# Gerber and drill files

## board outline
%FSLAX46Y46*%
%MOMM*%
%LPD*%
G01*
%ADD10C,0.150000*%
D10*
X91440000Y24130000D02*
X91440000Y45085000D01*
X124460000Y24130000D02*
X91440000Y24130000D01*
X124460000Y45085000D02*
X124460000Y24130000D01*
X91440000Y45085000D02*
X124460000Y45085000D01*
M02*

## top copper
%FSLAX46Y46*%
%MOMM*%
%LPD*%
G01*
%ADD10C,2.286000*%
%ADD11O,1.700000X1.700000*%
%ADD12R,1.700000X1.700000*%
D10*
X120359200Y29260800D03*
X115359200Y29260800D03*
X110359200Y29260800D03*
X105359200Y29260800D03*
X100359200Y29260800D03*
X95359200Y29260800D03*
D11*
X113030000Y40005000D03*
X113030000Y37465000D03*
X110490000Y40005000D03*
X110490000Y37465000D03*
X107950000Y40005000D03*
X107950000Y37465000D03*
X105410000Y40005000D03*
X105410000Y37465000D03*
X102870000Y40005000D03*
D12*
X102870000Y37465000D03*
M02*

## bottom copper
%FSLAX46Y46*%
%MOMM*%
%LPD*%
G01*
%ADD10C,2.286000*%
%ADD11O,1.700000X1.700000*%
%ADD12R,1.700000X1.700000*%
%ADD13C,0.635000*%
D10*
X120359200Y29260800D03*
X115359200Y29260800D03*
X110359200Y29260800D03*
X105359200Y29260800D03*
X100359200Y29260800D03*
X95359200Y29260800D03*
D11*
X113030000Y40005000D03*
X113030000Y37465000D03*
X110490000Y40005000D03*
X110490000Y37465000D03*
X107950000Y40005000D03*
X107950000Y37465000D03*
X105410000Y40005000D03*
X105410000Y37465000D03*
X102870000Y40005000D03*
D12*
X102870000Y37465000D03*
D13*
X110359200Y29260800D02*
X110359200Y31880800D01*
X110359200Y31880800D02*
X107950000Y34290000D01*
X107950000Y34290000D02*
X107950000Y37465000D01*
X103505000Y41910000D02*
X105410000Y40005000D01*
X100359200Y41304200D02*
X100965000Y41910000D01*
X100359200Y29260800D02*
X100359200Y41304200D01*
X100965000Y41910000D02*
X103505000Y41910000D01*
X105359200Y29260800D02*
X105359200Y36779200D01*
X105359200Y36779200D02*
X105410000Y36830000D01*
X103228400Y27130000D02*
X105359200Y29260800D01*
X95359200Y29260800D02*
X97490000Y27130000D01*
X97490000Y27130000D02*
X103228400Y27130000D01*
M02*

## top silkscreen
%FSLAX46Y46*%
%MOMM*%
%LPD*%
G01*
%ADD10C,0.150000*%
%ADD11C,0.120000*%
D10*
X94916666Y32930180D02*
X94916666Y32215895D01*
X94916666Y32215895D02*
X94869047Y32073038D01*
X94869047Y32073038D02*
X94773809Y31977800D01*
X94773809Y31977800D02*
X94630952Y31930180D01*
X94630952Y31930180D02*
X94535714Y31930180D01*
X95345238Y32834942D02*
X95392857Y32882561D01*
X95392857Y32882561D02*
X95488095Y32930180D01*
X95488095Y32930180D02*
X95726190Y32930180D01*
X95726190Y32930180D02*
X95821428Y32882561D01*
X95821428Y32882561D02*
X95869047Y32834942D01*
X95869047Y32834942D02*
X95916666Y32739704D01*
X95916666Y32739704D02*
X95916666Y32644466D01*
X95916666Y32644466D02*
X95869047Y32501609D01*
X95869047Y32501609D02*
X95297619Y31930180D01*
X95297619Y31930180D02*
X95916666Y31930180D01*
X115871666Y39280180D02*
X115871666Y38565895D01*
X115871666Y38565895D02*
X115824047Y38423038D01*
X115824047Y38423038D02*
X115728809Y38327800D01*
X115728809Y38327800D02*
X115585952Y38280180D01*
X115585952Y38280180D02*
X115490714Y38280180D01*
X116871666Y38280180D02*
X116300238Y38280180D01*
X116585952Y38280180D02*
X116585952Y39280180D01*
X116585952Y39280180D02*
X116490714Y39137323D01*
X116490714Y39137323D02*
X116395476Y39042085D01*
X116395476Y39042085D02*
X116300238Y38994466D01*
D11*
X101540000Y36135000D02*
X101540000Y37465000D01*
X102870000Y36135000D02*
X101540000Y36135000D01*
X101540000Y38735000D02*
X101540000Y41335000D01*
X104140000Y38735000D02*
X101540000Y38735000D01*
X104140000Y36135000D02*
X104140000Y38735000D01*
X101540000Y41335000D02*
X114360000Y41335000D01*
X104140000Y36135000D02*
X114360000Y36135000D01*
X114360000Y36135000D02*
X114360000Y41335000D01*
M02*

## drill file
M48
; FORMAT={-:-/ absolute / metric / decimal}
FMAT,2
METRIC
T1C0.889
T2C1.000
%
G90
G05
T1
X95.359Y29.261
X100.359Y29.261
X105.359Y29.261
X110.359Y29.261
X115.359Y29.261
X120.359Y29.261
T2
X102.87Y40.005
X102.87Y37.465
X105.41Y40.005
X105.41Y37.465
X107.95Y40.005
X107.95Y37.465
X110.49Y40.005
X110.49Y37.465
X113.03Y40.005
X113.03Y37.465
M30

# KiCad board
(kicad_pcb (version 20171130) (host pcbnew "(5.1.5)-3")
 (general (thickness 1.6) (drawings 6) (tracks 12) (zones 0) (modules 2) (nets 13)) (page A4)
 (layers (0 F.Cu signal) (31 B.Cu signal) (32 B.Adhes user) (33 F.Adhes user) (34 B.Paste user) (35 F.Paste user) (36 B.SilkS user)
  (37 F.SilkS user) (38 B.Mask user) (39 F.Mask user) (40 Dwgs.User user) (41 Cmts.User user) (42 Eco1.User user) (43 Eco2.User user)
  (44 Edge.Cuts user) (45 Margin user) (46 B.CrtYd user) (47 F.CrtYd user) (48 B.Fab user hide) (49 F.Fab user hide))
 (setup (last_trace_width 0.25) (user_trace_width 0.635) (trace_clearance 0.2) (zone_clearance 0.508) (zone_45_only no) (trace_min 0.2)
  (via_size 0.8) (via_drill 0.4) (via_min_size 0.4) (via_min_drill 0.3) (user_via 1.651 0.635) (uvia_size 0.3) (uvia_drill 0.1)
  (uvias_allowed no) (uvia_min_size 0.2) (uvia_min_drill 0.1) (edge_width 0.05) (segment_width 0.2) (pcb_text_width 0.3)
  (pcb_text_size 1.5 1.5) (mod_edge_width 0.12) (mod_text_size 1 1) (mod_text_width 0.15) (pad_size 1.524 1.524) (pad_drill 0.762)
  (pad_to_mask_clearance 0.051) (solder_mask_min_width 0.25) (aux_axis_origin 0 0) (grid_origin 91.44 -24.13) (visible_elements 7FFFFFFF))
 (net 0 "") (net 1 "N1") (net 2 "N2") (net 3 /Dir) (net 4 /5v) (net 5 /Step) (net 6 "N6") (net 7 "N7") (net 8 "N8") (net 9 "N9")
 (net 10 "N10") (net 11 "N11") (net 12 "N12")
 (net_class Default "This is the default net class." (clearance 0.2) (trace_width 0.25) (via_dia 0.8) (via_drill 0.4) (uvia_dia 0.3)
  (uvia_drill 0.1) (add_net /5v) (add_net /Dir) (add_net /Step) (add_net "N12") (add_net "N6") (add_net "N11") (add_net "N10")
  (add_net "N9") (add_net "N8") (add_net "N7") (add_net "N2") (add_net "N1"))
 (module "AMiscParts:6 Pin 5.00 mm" (layer F.Cu) (at 107.8592 -29.2608)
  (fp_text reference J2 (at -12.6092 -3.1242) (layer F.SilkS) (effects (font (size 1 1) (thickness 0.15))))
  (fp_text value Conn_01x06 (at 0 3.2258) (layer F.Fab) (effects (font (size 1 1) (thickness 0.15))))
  (pad 6 thru_hole circle (at 12.5 0) (size 2.286 2.286) (drill 0.889) (layers *.Cu *.Mask) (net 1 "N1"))
  (pad 5 thru_hole circle (at 7.5 0) (size 2.286 2.286) (drill 0.889) (layers *.Cu *.Mask) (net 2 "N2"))
  (pad 4 thru_hole circle (at 2.5 0) (size 2.286 2.286) (drill 0.889) (layers *.Cu *.Mask) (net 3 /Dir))
  (pad 3 thru_hole circle (at -2.5 0) (size 2.286 2.286) (drill 0.889) (layers *.Cu *.Mask) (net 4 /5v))
  (pad 2 thru_hole circle (at -7.5 0) (size 2.286 2.286) (drill 0.889) (layers *.Cu *.Mask) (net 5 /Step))
  (pad 1 thru_hole circle (at -12.5 0) (size 2.286 2.286) (drill 0.889) (layers *.Cu *.Mask) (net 4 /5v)))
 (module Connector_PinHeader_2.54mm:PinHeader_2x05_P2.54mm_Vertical (layer F.Cu) (at 102.87 -37.465 90)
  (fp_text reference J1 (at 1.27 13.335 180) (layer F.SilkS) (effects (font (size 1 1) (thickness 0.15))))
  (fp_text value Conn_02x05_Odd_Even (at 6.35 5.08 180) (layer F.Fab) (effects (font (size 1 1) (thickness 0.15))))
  (fp_line (start -1.33 -1.33) (end 0 -1.33) (layer F.SilkS) (width 0.12))
  (fp_line (start -1.33 0) (end -1.33 -1.33) (layer F.SilkS) (width 0.12))
  (fp_line (start 1.27 -1.33) (end 3.87 -1.33) (layer F.SilkS) (width 0.12))
  (fp_line (start 1.27 1.27) (end 1.27 -1.33) (layer F.SilkS) (width 0.12))
  (fp_line (start -1.33 1.27) (end 1.27 1.27) (layer F.SilkS) (width 0.12))
  (fp_line (start 3.87 -1.33) (end 3.87 11.49) (layer F.SilkS) (width 0.12))
  (fp_line (start -1.33 1.27) (end -1.33 11.49) (layer F.SilkS) (width 0.12))
  (fp_line (start -1.33 11.49) (end 3.87 11.49) (layer F.SilkS) (width 0.12))
  (pad 10 thru_hole oval (at 2.54 10.16 90) (size 1.7 1.7) (drill 1) (layers *.Cu *.Mask) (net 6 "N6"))
  (pad 9 thru_hole oval (at 0 10.16 90) (size 1.7 1.7) (drill 1) (layers *.Cu *.Mask) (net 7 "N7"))
  (pad 8 thru_hole oval (at 2.54 7.62 90) (size 1.7 1.7) (drill 1) (layers *.Cu *.Mask) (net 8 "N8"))
  (pad 7 thru_hole oval (at 0 7.62 90) (size 1.7 1.7) (drill 1) (layers *.Cu *.Mask) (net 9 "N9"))
  (pad 6 thru_hole oval (at 2.54 5.08 90) (size 1.7 1.7) (drill 1) (layers *.Cu *.Mask) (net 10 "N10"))
  (pad 5 thru_hole oval (at 0 5.08 90) (size 1.7 1.7) (drill 1) (layers *.Cu *.Mask) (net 3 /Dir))
  (pad 4 thru_hole oval (at 2.54 2.54 90) (size 1.7 1.7) (drill 1) (layers *.Cu *.Mask) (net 5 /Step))
  (pad 3 thru_hole oval (at 0 2.54 90) (size 1.7 1.7) (drill 1) (layers *.Cu *.Mask) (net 4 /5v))
  (pad 2 thru_hole oval (at 2.54 0 90) (size 1.7 1.7) (drill 1) (layers *.Cu *.Mask) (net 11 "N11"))
  (pad 1 thru_hole rect (at 0 0 90) (size 1.7 1.7) (drill 1) (layers *.Cu *.Mask) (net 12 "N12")))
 (gr_line (start 91.44 -24.13) (end 91.44 -45.085) (layer Edge.Cuts) (width 0.15))
 (gr_line (start 124.46 -24.13) (end 91.44 -24.13) (layer Edge.Cuts) (width 0.15))
 (gr_line (start 124.46 -45.085) (end 124.46 -24.13) (layer Edge.Cuts) (width 0.15))
 (gr_line (start 91.44 -45.085) (end 124.46 -45.085) (layer Edge.Cuts) (width 0.15))
 (segment (start 110.3592 -29.2608) (end 110.3592 -31.8808) (width 0.635) (layer B.Cu) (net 3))
 (segment (start 110.3592 -31.8808) (end 107.95 -34.29) (width 0.635) (layer B.Cu) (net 3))
 (segment (start 107.95 -34.29) (end 107.95 -37.465) (width 0.635) (layer B.Cu) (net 3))
 (segment (start 103.505 -41.91) (end 105.41 -40.005) (width 0.635) (layer B.Cu) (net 5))
 (segment (start 100.3592 -41.3042) (end 100.965 -41.91) (width 0.635) (layer B.Cu) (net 5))
 (segment (start 100.3592 -29.2608) (end 100.3592 -41.3042) (width 0.635) (layer B.Cu) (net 5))
 (segment (start 100.965 -41.91) (end 103.505 -41.91) (width 0.635) (layer B.Cu) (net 5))
 (segment (start 105.3592 -29.2608) (end 105.3592 -36.7792) (width 0.635) (layer B.Cu) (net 4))
 (segment (start 105.3592 -36.7792) (end 105.41 -36.83) (width 0.635) (layer B.Cu) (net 4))
 (segment (start 103.2284 -27.13) (end 105.3592 -29.2608) (width 0.635) (layer B.Cu) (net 4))
 (segment (start 95.3592 -29.2608) (end 97.49 -27.13) (width 0.635) (layer B.Cu) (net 4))
 (segment (start 97.49 -27.13) (end 103.2284 -27.13) (width 0.635) (layer B.Cu) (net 4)))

